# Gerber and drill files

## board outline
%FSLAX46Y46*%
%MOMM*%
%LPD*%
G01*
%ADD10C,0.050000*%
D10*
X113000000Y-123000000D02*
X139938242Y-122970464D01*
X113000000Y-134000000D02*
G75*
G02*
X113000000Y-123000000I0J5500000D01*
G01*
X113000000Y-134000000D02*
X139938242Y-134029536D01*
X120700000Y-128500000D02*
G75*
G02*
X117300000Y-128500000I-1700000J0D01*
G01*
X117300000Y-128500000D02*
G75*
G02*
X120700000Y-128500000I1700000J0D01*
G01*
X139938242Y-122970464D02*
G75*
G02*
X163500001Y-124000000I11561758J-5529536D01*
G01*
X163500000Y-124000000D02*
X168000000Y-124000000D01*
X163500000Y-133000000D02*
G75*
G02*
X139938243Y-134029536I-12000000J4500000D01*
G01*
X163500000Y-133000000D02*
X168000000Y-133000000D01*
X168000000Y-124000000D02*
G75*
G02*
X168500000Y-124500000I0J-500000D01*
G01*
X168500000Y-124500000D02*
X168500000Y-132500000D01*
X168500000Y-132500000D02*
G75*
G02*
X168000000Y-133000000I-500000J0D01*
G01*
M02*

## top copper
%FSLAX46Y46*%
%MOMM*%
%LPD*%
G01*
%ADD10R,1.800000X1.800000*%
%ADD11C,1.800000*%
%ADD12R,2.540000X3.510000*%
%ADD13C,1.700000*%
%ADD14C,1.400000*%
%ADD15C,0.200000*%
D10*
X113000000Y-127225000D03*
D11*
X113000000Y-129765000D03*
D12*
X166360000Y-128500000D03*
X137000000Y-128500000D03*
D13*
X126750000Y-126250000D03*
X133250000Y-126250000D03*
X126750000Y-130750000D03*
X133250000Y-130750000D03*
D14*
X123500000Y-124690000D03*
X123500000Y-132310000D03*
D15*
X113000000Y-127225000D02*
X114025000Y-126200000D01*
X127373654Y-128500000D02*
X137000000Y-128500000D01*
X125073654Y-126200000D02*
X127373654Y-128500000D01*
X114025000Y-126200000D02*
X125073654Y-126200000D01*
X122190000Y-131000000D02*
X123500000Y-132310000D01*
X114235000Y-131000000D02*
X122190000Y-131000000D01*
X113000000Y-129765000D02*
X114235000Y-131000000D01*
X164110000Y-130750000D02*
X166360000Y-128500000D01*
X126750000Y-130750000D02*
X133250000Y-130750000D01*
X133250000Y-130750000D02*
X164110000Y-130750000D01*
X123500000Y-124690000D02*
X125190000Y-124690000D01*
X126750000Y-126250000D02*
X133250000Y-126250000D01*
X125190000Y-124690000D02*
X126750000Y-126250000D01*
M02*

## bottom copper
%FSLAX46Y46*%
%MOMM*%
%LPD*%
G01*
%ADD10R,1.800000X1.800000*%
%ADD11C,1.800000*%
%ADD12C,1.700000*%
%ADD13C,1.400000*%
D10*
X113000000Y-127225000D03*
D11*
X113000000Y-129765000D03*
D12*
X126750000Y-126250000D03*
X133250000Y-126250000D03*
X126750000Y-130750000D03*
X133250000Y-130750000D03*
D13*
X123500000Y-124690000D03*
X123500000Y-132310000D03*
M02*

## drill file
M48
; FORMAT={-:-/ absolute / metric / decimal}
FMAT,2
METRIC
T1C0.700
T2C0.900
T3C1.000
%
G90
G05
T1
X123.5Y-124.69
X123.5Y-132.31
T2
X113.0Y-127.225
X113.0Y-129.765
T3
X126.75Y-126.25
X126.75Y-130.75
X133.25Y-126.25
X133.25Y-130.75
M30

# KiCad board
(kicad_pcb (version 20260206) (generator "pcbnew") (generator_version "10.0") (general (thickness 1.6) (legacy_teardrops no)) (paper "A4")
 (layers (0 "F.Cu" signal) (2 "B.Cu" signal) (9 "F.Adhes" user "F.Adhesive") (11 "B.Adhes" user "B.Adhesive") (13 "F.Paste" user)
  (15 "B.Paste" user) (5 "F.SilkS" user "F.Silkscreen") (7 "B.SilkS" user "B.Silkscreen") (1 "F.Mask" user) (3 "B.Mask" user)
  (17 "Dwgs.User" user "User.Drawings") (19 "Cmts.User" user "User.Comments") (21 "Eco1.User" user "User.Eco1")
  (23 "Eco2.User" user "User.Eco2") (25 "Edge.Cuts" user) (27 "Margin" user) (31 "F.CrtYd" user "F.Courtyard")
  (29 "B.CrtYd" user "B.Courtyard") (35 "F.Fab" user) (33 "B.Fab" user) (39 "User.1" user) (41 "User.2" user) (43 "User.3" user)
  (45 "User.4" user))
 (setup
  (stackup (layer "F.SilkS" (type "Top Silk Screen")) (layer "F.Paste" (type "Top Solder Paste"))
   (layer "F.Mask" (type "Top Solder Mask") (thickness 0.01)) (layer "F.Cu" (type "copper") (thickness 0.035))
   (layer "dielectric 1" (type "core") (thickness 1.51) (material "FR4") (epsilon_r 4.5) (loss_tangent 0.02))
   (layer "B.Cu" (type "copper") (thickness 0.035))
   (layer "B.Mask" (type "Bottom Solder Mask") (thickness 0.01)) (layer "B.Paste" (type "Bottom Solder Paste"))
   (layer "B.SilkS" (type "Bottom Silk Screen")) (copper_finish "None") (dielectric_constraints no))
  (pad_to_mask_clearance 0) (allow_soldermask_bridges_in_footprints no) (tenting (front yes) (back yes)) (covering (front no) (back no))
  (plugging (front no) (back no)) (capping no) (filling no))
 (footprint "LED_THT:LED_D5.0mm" (layer "F.Cu") (at 113 127.225 -90)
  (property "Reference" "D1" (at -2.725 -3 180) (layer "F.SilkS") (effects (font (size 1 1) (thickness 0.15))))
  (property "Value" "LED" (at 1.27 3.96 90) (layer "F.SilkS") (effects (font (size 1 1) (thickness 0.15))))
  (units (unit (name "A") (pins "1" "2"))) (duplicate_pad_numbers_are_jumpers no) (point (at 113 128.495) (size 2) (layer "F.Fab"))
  (pad "1" thru_hole rect (at 0 0 270) (size 1.8 1.8) (drill 0.9) (layers "*.Cu" "*.Mask") (remove_unused_layers no) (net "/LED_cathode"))
  (pad "2" thru_hole circle (at 2.54 0 270) (size 1.8 1.8) (drill 0.9) (layers "*.Cu" "*.Mask") (remove_unused_layers no) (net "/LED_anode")))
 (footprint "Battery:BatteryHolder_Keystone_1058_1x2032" (layer "F.Cu") (at 151.68 128.5 180)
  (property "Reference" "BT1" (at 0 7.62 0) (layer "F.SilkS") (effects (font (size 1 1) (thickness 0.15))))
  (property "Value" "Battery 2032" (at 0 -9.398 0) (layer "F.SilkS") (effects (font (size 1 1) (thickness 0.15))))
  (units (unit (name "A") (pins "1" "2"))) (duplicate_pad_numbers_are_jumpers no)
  (pad "1" smd rect (at -14.68 0 180) (size 2.54 3.51) (layers "F.Cu" "F.Mask" "F.Paste") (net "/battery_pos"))
  (pad "2" smd rect (at 14.68 0 180) (size 2.54 3.51) (layers "F.Cu" "F.Mask" "F.Paste") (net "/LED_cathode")))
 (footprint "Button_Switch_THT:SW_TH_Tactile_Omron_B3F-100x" (layer "F.Cu") (at 126.75 126.25)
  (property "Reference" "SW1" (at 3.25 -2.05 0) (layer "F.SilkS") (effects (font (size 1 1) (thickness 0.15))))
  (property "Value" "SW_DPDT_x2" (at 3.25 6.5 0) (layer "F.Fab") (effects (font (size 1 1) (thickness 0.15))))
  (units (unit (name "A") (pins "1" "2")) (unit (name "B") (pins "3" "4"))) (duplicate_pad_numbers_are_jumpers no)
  (pad "1" thru_hole circle (at 0 0) (size 1.7 1.7) (drill 1) (layers "*.Cu" "*.Mask") (remove_unused_layers no) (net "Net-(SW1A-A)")
   (thermal_bridge_angle 90))
  (pad "1" thru_hole circle (at 6.5 0) (size 1.7 1.7) (drill 1) (layers "*.Cu" "*.Mask") (remove_unused_layers no) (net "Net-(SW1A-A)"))
  (pad "2" thru_hole circle (at 0 4.5) (size 1.7 1.7) (drill 1) (layers "*.Cu" "*.Mask") (remove_unused_layers no) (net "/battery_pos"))
  (pad "2" thru_hole circle (at 6.5 4.5) (size 1.7 1.7) (drill 1) (layers "*.Cu" "*.Mask") (remove_unused_layers no) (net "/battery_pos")))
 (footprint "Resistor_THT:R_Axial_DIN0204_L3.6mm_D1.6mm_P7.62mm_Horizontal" (layer "F.Cu") (at 123.5 124.69 -90)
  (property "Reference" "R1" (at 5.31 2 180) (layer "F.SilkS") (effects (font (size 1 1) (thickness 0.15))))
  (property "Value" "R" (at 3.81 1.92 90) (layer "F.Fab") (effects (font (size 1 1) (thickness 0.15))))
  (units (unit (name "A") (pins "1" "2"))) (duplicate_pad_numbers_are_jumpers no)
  (pad "1" thru_hole circle (at 0 0 270) (size 1.4 1.4) (drill 0.7) (layers "*.Cu" "*.Mask") (remove_unused_layers no) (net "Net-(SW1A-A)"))
  (pad "2" thru_hole circle (at 7.62 0 270) (size 1.4 1.4) (drill 0.7) (layers "*.Cu" "*.Mask") (remove_unused_layers no) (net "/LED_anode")))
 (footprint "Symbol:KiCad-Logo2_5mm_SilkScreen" (layer "B.Cu") (at 151 127.5 180)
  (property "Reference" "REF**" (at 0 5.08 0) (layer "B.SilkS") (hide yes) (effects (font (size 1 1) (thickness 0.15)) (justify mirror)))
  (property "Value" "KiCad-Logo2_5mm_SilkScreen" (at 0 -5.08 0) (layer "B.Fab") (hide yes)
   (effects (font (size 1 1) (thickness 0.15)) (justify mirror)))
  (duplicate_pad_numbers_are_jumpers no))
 (gr_line (start 113 123) (end 139.938242 122.970464) (stroke (width 0.05) (type default)) (locked yes) (layer "Edge.Cuts"))
 (gr_arc (start 113 134) (mid 107.5 128.5) (end 113 123) (stroke (width 0.05) (type default)) (locked yes) (layer "Edge.Cuts"))
 (gr_line (start 113 134) (end 139.938242 134.029536) (stroke (width 0.05) (type default)) (locked yes) (layer "Edge.Cuts"))
 (gr_circle (center 119 128.5) (end 120.7 128.5) (stroke (width 0.05) (type solid)) (fill no) (layer "Edge.Cuts"))
 (gr_arc (start 139.938242 122.970464) (mid 152.059464 115.696211) (end 163.5 124) (stroke (width 0.05) (type default)) (locked yes)
  (layer "Edge.Cuts"))
 (gr_line (start 163.5 124) (end 168 124) (stroke (width 0.05) (type default)) (locked yes) (layer "Edge.Cuts"))
 (gr_arc (start 163.5 133) (mid 152.059464 141.303788) (end 139.938242 134.029536) (stroke (width 0.05) (type default)) (locked yes)
  (layer "Edge.Cuts"))
 (gr_line (start 163.5 133) (end 168 133) (stroke (width 0.05) (type default)) (locked yes) (layer "Edge.Cuts"))
 (gr_arc (start 168 124) (mid 168.353553 124.146447) (end 168.5 124.5) (stroke (width 0.05) (type default)) (locked yes) (layer "Edge.Cuts"))
 (gr_line (start 168.5 124.5) (end 168.5 132.5) (stroke (width 0.05) (type default)) (locked yes) (layer "Edge.Cuts"))
 (gr_arc (start 168.5 132.5) (mid 168.353553 132.853553) (end 168 133) (stroke (width 0.05) (type default)) (locked yes) (layer "Edge.Cuts"))
 (segment (start 113 127.225) (end 114.025 126.2) (width 0.2) (layer "F.Cu") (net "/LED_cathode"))
 (segment (start 127.373654 128.5) (end 137 128.5) (width 0.2) (layer "F.Cu") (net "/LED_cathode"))
 (segment (start 125.073654 126.2) (end 127.373654 128.5) (width 0.2) (layer "F.Cu") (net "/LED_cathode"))
 (segment (start 114.025 126.2) (end 125.073654 126.2) (width 0.2) (layer "F.Cu") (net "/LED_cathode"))
 (segment (start 122.19 131) (end 123.5 132.31) (width 0.2) (layer "F.Cu") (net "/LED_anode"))
 (segment (start 114.235 131) (end 122.19 131) (width 0.2) (layer "F.Cu") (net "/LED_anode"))
 (segment (start 113 129.765) (end 114.235 131) (width 0.2) (layer "F.Cu") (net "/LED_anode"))
 (segment (start 164.11 130.75) (end 166.36 128.5) (width 0.2) (layer "F.Cu") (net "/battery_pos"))
 (segment (start 126.75 130.75) (end 133.25 130.75) (width 0.2) (layer "F.Cu") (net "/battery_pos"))
 (segment (start 133.25 130.75) (end 164.11 130.75) (width 0.2) (layer "F.Cu") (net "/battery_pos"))
 (segment (start 123.5 124.69) (end 125.19 124.69) (width 0.2) (layer "F.Cu") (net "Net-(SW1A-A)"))
 (segment (start 126.75 126.25) (end 133.25 126.25) (width 0.2) (layer "F.Cu") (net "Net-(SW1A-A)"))
 (segment (start 125.19 124.69) (end 126.75 126.25) (width 0.2) (layer "F.Cu") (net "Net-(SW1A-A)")))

